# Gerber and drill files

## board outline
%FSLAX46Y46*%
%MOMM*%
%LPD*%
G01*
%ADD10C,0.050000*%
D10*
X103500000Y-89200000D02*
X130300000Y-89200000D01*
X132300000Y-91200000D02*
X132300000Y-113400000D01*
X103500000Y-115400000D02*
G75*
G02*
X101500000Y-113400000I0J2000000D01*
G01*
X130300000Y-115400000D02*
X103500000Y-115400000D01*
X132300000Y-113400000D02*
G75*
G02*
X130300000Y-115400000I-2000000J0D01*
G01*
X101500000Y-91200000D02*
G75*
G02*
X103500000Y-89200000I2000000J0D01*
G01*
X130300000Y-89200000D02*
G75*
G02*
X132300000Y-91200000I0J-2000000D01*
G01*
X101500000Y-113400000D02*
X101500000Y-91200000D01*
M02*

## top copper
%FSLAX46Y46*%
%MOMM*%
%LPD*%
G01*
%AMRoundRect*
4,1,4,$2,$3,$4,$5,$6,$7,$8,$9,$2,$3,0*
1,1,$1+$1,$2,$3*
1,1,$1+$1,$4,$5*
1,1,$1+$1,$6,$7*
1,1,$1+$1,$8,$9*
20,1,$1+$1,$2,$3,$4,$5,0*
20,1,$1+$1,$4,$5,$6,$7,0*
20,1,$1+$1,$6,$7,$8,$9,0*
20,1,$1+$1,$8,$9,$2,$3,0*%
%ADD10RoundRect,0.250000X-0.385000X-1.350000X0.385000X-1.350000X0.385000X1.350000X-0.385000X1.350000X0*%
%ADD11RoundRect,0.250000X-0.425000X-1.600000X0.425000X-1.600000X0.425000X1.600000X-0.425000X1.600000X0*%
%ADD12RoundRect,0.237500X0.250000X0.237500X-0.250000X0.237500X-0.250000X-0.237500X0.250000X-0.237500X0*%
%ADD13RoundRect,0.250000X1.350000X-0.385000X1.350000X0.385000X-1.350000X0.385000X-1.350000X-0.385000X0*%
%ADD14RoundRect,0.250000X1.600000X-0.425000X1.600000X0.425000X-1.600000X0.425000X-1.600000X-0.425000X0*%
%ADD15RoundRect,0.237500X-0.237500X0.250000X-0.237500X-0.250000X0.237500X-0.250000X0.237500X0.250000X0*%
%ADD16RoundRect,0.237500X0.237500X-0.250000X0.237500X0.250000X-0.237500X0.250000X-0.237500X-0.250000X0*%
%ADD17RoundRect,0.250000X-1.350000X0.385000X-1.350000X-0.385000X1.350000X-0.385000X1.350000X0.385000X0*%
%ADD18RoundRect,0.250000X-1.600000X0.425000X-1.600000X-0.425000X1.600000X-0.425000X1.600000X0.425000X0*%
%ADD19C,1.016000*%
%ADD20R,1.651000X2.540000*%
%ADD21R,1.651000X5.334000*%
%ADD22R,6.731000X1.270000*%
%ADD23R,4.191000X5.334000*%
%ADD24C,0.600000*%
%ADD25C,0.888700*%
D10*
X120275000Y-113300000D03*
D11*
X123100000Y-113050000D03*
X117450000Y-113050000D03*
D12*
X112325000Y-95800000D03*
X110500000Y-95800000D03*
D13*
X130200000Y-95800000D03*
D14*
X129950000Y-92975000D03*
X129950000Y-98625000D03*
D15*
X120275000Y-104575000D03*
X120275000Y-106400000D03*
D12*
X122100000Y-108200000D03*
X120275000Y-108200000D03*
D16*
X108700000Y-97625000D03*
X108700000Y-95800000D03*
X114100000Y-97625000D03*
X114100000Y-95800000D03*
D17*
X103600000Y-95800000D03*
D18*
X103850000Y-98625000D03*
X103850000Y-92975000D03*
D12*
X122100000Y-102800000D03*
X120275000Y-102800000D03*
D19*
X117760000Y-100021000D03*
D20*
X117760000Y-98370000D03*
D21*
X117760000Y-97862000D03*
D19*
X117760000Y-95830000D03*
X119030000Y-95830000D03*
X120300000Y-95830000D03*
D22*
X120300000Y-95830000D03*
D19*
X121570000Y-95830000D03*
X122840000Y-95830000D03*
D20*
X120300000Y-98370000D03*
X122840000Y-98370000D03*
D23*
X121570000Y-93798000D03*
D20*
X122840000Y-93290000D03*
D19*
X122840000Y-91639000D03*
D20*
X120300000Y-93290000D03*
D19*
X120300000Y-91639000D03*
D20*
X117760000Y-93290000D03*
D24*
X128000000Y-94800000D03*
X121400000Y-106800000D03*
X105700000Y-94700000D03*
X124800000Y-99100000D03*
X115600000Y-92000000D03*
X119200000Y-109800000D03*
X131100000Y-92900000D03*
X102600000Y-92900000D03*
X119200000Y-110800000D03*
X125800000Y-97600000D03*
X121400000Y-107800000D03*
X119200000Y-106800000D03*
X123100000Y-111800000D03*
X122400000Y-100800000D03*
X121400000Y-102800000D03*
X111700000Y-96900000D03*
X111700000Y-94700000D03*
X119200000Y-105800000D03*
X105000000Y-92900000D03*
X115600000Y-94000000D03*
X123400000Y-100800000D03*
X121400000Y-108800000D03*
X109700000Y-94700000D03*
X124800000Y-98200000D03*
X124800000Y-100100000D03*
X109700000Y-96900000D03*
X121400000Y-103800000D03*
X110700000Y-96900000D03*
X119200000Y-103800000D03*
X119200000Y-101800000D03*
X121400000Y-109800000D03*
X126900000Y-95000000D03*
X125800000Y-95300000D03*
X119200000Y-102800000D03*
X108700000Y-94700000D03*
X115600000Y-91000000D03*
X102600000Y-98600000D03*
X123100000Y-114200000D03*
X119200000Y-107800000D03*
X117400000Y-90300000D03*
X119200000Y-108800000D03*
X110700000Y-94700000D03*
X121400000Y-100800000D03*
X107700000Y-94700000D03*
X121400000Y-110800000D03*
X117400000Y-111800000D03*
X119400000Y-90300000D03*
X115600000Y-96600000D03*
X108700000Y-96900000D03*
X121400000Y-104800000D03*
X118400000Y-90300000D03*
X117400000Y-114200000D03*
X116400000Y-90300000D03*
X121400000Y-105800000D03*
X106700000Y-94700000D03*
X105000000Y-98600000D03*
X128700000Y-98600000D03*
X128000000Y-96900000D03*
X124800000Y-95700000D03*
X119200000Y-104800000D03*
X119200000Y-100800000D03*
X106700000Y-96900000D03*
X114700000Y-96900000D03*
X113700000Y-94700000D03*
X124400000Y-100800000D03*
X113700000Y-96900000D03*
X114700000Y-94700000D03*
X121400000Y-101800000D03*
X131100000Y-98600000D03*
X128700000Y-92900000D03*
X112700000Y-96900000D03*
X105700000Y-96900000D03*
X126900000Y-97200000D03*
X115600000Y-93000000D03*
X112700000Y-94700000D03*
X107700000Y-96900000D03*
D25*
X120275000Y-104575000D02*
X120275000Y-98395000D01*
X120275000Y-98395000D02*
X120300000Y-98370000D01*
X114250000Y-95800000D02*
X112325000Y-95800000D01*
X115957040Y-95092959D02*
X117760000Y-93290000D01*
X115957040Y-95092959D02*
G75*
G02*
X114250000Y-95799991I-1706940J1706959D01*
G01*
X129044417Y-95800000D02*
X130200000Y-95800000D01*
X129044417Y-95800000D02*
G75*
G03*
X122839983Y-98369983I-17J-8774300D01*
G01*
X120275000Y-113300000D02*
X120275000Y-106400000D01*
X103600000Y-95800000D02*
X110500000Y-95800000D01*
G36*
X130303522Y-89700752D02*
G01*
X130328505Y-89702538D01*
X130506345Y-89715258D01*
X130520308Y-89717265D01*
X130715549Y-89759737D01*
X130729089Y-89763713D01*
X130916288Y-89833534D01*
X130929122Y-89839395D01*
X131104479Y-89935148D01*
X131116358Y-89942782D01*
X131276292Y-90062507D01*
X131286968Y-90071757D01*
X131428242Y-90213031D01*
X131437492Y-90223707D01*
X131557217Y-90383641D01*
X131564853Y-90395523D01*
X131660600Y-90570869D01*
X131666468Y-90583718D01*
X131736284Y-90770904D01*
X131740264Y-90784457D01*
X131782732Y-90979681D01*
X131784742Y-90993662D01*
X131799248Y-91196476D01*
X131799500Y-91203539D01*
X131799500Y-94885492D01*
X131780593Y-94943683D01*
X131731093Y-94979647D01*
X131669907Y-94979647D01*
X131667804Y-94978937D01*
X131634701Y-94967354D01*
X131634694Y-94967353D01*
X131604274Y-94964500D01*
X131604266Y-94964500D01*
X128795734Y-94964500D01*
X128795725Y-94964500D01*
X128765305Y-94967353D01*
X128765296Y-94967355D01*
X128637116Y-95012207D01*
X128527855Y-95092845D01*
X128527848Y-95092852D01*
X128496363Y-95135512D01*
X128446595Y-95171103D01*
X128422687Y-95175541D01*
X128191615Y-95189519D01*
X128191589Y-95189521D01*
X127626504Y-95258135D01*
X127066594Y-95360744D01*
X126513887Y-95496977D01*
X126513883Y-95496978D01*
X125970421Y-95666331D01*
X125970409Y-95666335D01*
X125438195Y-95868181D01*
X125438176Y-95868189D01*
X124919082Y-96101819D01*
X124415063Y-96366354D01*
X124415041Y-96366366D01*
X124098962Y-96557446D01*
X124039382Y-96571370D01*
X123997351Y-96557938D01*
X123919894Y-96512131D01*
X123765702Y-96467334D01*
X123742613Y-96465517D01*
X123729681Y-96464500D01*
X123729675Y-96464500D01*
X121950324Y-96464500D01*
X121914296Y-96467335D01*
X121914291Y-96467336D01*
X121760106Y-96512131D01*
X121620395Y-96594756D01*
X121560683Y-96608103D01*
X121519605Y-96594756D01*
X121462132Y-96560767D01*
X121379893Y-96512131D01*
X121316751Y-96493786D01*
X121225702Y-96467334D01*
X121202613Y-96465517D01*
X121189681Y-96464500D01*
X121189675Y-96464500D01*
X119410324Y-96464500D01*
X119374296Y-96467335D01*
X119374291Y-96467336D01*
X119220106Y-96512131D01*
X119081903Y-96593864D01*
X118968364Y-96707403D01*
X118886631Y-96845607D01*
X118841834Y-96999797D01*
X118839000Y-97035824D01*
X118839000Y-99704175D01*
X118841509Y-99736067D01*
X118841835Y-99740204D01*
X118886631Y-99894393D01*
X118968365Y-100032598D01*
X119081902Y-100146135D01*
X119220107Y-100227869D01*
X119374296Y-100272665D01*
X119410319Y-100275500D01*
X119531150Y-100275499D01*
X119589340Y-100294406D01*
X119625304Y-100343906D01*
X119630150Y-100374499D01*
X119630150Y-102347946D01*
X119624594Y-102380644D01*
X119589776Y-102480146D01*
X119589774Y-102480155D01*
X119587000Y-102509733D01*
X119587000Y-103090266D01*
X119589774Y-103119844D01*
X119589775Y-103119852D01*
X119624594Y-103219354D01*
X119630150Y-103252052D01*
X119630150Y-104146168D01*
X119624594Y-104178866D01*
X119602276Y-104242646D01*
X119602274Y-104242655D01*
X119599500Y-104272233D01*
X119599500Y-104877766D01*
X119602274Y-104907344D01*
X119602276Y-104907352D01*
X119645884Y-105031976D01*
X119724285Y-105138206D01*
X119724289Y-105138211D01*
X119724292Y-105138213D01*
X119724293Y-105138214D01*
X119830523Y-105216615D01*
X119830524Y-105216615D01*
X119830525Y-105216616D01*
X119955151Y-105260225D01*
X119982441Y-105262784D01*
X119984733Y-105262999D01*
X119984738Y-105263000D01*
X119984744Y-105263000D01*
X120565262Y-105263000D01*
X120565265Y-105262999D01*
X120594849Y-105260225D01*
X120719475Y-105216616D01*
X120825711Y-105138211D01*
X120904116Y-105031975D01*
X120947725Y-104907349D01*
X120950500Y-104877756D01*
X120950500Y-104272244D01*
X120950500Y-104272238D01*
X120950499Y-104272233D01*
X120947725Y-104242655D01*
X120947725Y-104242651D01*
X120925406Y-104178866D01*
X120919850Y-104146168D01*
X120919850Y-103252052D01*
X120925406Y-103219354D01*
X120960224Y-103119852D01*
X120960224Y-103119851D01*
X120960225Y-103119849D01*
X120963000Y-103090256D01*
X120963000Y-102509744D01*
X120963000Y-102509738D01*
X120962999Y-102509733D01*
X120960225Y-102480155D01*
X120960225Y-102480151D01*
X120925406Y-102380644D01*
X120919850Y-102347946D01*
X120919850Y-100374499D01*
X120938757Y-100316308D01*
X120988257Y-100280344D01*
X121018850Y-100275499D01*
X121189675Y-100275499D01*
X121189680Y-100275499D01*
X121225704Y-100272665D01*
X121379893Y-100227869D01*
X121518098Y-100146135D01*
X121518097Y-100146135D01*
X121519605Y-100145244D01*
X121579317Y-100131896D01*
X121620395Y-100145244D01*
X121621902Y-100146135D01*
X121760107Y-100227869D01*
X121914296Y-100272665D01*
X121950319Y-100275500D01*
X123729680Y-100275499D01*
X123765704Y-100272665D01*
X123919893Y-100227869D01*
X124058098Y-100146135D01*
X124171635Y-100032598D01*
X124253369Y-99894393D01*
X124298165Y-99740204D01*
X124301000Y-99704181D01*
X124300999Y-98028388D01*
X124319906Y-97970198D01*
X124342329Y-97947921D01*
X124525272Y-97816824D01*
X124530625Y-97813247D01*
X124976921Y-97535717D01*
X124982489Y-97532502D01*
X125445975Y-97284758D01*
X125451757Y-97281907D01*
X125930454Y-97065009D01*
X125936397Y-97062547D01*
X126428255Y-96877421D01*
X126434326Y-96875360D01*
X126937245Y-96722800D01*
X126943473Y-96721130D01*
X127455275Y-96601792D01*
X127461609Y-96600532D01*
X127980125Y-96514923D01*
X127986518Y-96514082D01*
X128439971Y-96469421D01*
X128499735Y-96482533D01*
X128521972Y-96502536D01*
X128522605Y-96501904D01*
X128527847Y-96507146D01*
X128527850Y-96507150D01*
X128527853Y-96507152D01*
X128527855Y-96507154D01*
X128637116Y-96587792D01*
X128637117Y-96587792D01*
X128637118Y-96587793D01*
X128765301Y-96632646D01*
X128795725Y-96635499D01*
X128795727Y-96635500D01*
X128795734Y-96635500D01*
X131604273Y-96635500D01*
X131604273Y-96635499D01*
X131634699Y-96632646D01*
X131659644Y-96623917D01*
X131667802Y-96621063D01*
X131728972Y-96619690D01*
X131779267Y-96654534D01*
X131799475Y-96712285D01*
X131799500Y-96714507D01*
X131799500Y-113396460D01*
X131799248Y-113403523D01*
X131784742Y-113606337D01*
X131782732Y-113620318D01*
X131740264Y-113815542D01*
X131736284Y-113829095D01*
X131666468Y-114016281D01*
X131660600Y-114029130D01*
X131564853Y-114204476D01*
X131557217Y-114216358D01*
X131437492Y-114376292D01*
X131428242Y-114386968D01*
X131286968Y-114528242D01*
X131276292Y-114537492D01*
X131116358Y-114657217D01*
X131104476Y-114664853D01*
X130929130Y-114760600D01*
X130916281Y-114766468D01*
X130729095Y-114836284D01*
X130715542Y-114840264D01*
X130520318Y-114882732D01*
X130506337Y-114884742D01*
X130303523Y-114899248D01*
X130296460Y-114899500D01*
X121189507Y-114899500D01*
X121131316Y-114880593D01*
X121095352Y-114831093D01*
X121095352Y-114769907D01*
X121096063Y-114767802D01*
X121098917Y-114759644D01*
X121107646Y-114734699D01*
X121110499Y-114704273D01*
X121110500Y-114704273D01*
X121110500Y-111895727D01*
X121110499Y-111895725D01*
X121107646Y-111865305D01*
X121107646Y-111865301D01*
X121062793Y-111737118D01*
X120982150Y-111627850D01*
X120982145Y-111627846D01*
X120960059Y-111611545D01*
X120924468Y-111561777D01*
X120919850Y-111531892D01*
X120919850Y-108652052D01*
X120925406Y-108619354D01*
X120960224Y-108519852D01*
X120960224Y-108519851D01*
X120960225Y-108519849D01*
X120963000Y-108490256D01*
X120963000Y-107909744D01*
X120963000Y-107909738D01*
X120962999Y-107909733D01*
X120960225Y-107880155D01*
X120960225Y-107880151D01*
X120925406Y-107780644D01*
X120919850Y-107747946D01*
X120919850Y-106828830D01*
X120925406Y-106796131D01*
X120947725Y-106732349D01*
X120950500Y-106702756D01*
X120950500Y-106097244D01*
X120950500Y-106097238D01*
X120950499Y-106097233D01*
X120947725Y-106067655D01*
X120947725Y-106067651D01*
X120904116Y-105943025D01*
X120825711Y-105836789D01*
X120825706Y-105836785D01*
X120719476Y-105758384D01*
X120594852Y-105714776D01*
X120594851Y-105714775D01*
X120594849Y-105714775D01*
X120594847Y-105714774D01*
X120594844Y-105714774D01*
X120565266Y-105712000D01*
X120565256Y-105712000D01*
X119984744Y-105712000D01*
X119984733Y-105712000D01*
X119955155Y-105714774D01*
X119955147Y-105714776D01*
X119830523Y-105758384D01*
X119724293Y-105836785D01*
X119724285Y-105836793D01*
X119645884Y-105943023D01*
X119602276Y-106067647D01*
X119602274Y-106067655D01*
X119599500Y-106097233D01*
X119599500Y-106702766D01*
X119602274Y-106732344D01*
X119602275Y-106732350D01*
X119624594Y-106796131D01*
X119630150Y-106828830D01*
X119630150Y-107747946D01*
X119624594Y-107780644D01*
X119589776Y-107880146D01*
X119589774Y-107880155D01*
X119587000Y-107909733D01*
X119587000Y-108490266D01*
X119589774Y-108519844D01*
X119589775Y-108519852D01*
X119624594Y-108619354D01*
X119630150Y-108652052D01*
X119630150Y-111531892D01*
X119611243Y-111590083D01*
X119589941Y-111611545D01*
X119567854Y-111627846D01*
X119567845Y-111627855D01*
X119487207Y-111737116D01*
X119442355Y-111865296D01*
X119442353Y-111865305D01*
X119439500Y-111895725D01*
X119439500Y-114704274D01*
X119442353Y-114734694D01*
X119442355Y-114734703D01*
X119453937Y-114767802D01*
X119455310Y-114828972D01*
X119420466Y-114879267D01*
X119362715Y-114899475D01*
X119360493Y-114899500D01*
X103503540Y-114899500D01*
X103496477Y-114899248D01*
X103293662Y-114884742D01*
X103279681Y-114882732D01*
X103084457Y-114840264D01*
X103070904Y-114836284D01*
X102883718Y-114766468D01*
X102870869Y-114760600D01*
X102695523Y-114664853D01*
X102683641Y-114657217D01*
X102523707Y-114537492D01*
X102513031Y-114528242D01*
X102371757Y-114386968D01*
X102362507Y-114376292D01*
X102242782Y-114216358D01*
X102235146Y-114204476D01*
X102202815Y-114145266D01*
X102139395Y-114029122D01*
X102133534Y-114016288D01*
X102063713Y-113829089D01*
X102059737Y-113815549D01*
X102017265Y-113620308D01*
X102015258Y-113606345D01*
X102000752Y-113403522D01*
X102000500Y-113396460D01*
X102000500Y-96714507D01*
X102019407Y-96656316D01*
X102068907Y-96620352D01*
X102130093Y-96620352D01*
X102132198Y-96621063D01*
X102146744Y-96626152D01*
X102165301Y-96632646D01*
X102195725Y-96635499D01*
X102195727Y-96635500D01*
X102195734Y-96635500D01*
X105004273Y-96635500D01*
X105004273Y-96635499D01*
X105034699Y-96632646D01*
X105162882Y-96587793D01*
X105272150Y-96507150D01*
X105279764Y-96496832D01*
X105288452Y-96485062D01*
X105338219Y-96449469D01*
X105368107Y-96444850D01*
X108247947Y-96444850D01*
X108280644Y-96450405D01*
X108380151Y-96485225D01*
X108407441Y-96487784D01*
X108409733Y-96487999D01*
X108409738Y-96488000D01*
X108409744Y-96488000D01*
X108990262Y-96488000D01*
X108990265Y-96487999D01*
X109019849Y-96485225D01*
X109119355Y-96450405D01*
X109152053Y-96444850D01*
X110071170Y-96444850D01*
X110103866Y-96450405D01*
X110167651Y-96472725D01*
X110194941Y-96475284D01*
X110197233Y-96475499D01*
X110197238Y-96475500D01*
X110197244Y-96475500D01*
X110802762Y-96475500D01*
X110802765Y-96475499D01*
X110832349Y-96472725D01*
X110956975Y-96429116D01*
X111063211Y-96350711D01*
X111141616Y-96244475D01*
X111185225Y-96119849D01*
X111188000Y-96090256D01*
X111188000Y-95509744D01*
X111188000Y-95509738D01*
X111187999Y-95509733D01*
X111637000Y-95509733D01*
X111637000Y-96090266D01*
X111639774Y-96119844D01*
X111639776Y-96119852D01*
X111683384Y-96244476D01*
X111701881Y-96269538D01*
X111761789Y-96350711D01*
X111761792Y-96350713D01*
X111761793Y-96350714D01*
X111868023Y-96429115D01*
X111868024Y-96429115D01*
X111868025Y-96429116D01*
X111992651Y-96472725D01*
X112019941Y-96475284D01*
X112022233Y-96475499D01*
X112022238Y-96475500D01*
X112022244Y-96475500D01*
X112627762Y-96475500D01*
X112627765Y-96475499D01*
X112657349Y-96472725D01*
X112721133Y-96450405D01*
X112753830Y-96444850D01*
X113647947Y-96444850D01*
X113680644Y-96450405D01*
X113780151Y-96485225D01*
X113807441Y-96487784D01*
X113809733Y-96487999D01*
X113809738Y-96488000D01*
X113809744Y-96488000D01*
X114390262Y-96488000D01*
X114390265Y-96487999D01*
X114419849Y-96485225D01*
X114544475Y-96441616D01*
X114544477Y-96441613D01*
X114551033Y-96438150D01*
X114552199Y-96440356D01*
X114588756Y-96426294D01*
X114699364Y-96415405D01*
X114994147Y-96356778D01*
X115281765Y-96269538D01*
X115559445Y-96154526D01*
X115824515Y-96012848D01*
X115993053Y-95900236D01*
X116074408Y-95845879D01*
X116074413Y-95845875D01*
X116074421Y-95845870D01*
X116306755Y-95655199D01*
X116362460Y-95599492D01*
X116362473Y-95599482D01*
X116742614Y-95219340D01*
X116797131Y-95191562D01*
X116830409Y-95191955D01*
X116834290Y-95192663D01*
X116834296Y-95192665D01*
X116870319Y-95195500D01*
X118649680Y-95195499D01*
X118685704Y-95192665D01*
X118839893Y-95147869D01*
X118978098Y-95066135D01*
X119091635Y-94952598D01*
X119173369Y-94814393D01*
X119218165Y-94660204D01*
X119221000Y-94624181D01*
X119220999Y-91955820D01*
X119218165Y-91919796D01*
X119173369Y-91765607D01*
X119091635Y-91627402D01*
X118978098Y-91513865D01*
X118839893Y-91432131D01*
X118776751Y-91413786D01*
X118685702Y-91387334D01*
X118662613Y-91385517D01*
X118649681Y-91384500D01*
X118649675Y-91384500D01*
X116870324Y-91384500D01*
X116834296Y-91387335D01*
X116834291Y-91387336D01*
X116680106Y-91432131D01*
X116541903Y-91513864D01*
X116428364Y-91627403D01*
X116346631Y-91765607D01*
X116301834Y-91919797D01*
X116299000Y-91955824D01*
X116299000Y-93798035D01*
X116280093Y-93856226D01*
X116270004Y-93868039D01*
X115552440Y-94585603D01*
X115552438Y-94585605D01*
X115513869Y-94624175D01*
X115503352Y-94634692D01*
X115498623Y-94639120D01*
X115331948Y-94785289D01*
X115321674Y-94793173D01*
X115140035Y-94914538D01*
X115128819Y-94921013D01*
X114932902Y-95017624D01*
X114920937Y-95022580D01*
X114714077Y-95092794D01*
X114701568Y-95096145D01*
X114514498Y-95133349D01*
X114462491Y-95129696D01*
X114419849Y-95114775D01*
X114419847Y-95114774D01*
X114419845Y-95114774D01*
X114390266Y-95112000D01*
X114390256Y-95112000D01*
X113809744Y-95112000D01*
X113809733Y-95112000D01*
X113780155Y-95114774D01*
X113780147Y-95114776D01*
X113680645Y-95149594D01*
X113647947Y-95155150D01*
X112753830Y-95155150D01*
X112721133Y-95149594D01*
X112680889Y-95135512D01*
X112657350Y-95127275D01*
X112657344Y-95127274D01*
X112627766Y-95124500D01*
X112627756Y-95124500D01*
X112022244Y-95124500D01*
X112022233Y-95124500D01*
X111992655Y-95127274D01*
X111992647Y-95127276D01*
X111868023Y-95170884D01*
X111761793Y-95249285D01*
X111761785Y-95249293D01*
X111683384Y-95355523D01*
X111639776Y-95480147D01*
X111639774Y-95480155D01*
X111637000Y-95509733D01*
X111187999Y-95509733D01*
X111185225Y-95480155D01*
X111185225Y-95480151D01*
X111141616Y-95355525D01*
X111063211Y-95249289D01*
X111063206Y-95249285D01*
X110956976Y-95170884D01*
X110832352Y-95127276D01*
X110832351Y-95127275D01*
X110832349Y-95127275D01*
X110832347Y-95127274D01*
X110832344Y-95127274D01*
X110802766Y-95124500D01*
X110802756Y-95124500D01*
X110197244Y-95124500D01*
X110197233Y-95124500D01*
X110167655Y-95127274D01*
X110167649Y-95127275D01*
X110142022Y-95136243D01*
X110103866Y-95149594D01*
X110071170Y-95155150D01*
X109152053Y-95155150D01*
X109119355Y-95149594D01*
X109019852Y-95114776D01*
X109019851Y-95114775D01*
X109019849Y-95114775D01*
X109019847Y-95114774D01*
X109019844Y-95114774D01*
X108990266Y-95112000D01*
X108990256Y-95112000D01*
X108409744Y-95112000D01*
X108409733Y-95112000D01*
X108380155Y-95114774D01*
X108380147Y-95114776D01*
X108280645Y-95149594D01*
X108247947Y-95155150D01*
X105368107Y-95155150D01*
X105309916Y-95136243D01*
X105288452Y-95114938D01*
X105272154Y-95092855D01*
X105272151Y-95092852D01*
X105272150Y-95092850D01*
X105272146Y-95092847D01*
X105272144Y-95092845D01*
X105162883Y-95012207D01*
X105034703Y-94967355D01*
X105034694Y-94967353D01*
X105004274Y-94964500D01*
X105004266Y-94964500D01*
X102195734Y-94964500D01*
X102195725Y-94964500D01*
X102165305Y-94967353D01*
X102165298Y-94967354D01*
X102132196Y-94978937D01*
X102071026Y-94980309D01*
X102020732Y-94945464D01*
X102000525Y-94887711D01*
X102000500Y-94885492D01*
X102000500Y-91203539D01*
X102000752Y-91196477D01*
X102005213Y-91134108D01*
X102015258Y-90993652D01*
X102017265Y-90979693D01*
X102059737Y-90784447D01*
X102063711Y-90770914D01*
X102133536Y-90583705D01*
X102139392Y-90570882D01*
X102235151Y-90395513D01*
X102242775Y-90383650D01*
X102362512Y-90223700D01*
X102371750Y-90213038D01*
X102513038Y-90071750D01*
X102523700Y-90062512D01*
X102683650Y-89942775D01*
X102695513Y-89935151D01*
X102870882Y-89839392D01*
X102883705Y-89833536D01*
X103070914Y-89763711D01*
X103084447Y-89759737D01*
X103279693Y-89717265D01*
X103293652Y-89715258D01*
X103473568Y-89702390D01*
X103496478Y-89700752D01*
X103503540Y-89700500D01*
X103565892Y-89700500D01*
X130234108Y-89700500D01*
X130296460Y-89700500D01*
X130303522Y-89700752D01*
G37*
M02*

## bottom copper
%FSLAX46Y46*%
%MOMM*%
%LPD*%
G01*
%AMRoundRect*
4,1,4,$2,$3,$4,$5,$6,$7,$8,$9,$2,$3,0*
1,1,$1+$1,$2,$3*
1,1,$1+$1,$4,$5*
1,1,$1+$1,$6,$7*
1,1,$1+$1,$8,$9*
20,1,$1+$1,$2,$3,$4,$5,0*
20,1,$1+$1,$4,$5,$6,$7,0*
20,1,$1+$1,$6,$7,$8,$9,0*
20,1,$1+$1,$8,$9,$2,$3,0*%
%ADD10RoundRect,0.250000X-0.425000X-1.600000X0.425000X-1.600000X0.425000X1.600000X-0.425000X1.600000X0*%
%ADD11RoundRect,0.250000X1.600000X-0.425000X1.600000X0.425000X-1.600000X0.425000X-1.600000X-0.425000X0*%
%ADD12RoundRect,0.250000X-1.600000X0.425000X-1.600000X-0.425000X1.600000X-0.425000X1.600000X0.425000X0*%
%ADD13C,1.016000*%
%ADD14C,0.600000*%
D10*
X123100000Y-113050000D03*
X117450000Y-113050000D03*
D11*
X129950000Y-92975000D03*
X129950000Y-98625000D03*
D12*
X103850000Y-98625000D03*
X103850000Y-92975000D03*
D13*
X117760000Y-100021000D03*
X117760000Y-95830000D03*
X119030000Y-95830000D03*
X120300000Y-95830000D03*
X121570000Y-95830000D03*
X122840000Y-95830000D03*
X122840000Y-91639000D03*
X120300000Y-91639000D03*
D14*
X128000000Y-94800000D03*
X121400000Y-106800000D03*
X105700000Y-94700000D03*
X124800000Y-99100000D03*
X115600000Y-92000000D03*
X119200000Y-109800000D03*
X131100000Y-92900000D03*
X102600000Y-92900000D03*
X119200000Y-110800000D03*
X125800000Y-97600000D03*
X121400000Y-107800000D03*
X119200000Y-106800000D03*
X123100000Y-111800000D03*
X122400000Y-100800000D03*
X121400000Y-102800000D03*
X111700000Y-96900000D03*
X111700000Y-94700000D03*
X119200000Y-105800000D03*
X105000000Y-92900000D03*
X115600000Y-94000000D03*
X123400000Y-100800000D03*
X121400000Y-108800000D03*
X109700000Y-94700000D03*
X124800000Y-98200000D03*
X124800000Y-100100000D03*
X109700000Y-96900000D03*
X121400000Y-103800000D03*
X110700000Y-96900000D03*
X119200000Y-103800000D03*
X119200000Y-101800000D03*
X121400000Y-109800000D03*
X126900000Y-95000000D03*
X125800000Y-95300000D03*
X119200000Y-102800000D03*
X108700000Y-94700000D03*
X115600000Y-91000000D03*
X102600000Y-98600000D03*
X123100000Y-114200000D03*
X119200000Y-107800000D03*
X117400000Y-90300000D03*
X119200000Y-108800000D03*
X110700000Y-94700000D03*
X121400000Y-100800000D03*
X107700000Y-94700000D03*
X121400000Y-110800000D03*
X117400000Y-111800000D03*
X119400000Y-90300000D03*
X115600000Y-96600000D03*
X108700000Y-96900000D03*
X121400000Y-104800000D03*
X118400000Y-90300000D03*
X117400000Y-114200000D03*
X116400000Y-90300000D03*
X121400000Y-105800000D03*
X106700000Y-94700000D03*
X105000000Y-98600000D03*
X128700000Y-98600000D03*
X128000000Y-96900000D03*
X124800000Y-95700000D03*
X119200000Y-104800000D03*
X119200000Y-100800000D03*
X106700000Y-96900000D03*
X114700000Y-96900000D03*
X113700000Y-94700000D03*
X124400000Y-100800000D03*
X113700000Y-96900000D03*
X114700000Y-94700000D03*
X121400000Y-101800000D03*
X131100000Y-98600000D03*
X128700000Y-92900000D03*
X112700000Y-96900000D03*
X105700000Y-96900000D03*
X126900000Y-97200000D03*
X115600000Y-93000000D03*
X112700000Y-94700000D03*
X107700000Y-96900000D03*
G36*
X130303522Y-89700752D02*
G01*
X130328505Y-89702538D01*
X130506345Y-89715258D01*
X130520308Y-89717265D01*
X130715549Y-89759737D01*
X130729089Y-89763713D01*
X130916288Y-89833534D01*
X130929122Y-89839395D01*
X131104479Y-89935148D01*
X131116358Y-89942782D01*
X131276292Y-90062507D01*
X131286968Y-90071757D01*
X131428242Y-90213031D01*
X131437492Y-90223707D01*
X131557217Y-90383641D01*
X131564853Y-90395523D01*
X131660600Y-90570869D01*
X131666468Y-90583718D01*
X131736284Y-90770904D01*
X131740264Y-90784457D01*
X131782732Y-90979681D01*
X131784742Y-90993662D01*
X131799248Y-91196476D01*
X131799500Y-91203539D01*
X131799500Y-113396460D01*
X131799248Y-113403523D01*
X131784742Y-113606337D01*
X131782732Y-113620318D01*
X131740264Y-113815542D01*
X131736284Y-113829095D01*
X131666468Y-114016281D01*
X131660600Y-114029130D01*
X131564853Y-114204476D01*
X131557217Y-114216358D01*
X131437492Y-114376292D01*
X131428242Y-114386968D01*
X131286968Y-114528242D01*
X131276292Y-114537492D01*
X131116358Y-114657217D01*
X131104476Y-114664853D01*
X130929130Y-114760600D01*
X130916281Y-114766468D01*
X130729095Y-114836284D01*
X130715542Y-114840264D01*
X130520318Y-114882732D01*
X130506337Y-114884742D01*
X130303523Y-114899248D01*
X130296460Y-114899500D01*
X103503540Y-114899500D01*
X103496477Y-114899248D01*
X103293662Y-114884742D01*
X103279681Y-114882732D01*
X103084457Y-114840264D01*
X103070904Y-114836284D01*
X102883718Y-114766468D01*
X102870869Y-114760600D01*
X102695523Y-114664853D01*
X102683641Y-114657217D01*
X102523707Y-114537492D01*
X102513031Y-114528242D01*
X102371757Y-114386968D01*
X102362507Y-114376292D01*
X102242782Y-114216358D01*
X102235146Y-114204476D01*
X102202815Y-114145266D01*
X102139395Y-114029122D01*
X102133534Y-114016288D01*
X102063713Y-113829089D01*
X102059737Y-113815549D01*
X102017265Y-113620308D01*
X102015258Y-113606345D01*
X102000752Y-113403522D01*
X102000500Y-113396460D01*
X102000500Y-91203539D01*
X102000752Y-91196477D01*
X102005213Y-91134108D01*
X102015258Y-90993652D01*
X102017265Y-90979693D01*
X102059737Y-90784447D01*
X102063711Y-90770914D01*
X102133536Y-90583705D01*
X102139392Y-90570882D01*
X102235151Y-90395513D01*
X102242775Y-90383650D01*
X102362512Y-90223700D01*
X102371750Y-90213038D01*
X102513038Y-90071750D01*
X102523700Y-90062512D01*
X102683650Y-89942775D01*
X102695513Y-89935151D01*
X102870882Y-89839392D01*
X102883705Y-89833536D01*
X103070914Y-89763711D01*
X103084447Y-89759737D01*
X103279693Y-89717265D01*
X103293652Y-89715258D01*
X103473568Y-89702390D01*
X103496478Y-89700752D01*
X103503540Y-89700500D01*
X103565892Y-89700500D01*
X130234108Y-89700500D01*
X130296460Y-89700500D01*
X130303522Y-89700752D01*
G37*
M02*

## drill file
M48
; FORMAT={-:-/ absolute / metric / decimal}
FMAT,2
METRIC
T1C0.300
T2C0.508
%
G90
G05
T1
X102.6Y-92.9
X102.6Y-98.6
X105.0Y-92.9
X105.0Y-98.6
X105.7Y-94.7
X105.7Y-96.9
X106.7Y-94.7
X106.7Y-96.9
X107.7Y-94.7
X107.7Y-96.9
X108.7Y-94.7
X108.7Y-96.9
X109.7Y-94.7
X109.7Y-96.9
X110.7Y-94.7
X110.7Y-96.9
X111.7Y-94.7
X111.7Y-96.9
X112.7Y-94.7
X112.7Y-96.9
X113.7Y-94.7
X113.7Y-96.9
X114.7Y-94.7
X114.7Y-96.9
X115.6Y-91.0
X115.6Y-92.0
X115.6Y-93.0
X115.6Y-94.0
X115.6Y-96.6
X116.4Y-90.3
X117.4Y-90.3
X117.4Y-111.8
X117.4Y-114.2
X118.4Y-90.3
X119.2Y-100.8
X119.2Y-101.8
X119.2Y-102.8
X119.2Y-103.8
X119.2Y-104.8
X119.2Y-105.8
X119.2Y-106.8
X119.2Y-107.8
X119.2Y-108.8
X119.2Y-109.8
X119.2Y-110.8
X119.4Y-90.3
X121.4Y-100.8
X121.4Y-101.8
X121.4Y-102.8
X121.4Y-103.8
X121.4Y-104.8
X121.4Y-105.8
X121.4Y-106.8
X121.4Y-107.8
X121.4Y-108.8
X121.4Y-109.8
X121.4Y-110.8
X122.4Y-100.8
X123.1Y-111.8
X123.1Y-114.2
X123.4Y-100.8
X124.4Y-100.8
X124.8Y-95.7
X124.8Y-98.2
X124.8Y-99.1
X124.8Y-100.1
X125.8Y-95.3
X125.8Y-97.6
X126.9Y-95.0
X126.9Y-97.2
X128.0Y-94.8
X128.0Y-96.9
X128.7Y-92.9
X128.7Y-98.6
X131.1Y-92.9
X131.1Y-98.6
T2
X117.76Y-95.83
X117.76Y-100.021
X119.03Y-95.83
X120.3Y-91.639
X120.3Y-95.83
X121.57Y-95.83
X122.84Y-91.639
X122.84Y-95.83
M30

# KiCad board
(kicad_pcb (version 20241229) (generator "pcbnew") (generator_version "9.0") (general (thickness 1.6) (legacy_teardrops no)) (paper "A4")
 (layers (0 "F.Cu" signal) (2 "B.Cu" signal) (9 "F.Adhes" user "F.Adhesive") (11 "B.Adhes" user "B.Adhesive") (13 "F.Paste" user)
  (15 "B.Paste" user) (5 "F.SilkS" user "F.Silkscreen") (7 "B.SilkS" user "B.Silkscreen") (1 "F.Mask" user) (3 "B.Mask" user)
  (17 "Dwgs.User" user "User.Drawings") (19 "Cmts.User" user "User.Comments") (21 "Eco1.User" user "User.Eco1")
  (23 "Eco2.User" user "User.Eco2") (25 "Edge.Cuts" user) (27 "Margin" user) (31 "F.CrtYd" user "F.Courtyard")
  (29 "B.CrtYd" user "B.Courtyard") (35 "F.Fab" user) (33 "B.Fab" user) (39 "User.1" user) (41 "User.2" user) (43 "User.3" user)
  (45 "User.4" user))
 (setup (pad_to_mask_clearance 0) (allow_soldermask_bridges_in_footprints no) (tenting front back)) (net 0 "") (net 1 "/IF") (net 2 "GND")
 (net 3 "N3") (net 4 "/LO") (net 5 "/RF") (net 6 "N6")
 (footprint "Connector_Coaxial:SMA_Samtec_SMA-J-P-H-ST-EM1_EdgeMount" (layer "F.Cu") (at 120.275 113.3 -90)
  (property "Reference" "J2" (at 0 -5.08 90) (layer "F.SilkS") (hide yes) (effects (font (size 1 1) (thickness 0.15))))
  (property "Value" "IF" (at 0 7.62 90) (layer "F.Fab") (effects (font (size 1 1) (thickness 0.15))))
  (pad "1" smd roundrect (at 0 0) (size 1.27 3.2) (layers "F.Cu" "F.Mask") (roundrect_rratio 0.1968503937) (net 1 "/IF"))
  (pad "2" smd roundrect (at -0.25 -2.825) (size 1.35 3.7) (layers "F.Cu" "F.Mask") (roundrect_rratio 0.1851851852) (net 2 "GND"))
  (pad "2" smd roundrect (at -0.25 -2.825) (size 1.35 3.7) (layers "B.Cu" "B.Mask") (roundrect_rratio 0.1851851852) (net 2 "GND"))
  (pad "2" smd roundrect (at -0.25 2.825) (size 1.35 3.7) (layers "F.Cu" "F.Mask") (roundrect_rratio 0.1851851852) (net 2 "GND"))
  (pad "2" smd roundrect (at -0.25 2.825) (size 1.35 3.7) (layers "B.Cu" "B.Mask") (roundrect_rratio 0.1851851852) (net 2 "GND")))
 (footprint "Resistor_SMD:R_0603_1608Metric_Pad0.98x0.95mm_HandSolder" (layer "F.Cu") (at 111.4125 95.8 180)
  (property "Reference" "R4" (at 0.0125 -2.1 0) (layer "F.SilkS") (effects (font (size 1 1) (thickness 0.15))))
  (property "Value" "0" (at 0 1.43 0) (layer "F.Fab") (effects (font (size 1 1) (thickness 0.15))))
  (pad "1" smd roundrect (at -0.9125 0 180) (size 0.975 0.95) (layers "F.Cu" "F.Mask" "F.Paste") (roundrect_rratio 0.25) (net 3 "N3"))
  (pad "2" smd roundrect (at 0.9125 0 180) (size 0.975 0.95) (layers "F.Cu" "F.Mask" "F.Paste") (roundrect_rratio 0.25) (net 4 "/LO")))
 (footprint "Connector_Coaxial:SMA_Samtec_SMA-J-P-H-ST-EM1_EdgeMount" (layer "F.Cu") (at 130.2 95.8)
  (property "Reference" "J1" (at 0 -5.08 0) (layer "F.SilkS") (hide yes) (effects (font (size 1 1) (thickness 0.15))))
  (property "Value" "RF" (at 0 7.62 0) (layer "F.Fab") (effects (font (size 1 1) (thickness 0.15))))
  (pad "1" smd roundrect (at 0 0 90) (size 1.27 3.2) (layers "F.Cu" "F.Mask") (roundrect_rratio 0.1968503937) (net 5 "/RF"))
  (pad "2" smd roundrect (at -0.25 -2.825 90) (size 1.35 3.7) (layers "F.Cu" "F.Mask") (roundrect_rratio 0.1851851852) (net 2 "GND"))
  (pad "2" smd roundrect (at -0.25 -2.825 90) (size 1.35 3.7) (layers "B.Cu" "B.Mask") (roundrect_rratio 0.1851851852) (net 2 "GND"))
  (pad "2" smd roundrect (at -0.25 2.825 90) (size 1.35 3.7) (layers "F.Cu" "F.Mask") (roundrect_rratio 0.1851851852) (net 2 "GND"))
  (pad "2" smd roundrect (at -0.25 2.825 90) (size 1.35 3.7) (layers "B.Cu" "B.Mask") (roundrect_rratio 0.1851851852) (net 2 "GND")))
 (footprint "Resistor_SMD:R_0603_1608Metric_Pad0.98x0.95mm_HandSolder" (layer "F.Cu") (at 120.275 105.4875 -90)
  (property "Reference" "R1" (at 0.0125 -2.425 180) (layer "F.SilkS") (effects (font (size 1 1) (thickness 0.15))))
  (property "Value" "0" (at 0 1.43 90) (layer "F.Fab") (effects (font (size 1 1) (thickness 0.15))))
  (pad "1" smd roundrect (at -0.9125 0 270) (size 0.975 0.95) (layers "F.Cu" "F.Mask" "F.Paste") (roundrect_rratio 0.25) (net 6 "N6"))
  (pad "2" smd roundrect (at 0.9125 0 270) (size 0.975 0.95) (layers "F.Cu" "F.Mask" "F.Paste") (roundrect_rratio 0.25) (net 1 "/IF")))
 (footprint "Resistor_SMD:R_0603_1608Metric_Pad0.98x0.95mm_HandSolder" (layer "F.Cu") (at 121.1875 108.2 180)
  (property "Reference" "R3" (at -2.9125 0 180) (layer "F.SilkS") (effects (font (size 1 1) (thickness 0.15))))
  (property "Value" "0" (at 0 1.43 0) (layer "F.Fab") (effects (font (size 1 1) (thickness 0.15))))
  (pad "1" smd roundrect (at -0.9125 0 180) (size 0.975 0.95) (layers "F.Cu" "F.Mask" "F.Paste") (roundrect_rratio 0.25) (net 2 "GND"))
  (pad "2" smd roundrect (at 0.9125 0 180) (size 0.975 0.95) (layers "F.Cu" "F.Mask" "F.Paste") (roundrect_rratio 0.25) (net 1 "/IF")))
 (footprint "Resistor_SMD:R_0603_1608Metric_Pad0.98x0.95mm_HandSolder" (layer "F.Cu") (at 108.7 96.7125 90)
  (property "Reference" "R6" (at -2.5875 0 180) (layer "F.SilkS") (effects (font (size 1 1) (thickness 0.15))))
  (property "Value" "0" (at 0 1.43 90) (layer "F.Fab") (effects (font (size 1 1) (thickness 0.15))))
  (pad "1" smd roundrect (at -0.9125 0 90) (size 0.975 0.95) (layers "F.Cu" "F.Mask" "F.Paste") (roundrect_rratio 0.25) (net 2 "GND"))
  (pad "2" smd roundrect (at 0.9125 0 90) (size 0.975 0.95) (layers "F.Cu" "F.Mask" "F.Paste") (roundrect_rratio 0.25) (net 4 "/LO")))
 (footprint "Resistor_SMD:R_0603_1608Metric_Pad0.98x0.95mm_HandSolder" (layer "F.Cu") (at 114.1 96.7125 90)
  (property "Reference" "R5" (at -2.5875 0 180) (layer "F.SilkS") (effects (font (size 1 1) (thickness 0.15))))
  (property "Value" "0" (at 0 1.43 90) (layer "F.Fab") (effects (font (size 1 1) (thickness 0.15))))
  (pad "1" smd roundrect (at -0.9125 0 90) (size 0.975 0.95) (layers "F.Cu" "F.Mask" "F.Paste") (roundrect_rratio 0.25) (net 2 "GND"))
  (pad "2" smd roundrect (at 0.9125 0 90) (size 0.975 0.95) (layers "F.Cu" "F.Mask" "F.Paste") (roundrect_rratio 0.25) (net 3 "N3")))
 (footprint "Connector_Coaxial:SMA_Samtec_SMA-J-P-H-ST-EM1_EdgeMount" (layer "F.Cu") (at 103.6 95.8 180)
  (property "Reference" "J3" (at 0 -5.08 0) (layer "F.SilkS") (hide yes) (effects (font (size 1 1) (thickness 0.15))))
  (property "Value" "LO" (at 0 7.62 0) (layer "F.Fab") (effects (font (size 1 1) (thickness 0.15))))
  (pad "1" smd roundrect (at 0 0 270) (size 1.27 3.2) (layers "F.Cu" "F.Mask") (roundrect_rratio 0.1968503937) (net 4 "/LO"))
  (pad "2" smd roundrect (at -0.25 -2.825 270) (size 1.35 3.7) (layers "F.Cu" "F.Mask") (roundrect_rratio 0.1851851852) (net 2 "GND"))
  (pad "2" smd roundrect (at -0.25 -2.825 270) (size 1.35 3.7) (layers "B.Cu" "B.Mask") (roundrect_rratio 0.1851851852) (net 2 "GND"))
  (pad "2" smd roundrect (at -0.25 2.825 270) (size 1.35 3.7) (layers "F.Cu" "F.Mask") (roundrect_rratio 0.1851851852) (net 2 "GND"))
  (pad "2" smd roundrect (at -0.25 2.825 270) (size 1.35 3.7) (layers "B.Cu" "B.Mask") (roundrect_rratio 0.1851851852) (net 2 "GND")))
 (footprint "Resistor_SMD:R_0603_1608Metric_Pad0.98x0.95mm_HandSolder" (layer "F.Cu") (at 121.1875 102.8 180)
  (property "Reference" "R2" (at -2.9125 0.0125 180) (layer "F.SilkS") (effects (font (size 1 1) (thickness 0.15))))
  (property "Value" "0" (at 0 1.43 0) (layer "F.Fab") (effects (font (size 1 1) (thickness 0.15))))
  (pad "1" smd roundrect (at -0.9125 0 180) (size 0.975 0.95) (layers "F.Cu" "F.Mask" "F.Paste") (roundrect_rratio 0.25) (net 2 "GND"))
  (pad "2" smd roundrect (at 0.9125 0 180) (size 0.975 0.95) (layers "F.Cu" "F.Mask" "F.Paste") (roundrect_rratio 0.25) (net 6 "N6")))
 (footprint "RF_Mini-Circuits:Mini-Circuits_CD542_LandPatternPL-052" (layer "F.Cu") (at 120.3 95.83 90)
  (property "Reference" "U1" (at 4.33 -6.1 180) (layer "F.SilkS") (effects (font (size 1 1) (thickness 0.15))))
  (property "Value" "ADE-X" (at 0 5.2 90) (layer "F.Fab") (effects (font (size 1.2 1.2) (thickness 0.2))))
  (pad "1" thru_hole circle (at -4.191 -2.54 90) (size 1.016 1.016) (drill 0.508) (layers "*.Cu") (remove_unused_layers no) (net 2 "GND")
   (zone_connect 2))
  (pad "1" smd rect (at -2.54 -2.54 90) (size 2.54 1.651) (layers "F.Cu" "F.Mask" "F.Paste") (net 2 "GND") (zone_connect 2))
  (pad "1" smd rect (at -2.032 -2.54 90) (size 5.334 1.651) (layers "F.Cu") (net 2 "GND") (zone_connect 2))
  (pad "1" thru_hole circle (at 0 -2.54 90) (size 1.016 1.016) (drill 0.508) (layers "*.Cu") (remove_unused_layers no) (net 2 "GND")
   (zone_connect 2))
  (pad "1" thru_hole circle (at 0 -1.27 90) (size 1.016 1.016) (drill 0.508) (layers "*.Cu") (remove_unused_layers no) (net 2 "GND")
   (zone_connect 2))
  (pad "1" thru_hole circle (at 0 0 90) (size 1.016 1.016) (drill 0.508) (layers "*.Cu") (remove_unused_layers no) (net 2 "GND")
   (zone_connect 2))
  (pad "1" smd rect (at 0 0 90) (size 1.27 6.731) (layers "F.Cu") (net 2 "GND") (zone_connect 2))
  (pad "1" thru_hole circle (at 0 1.27 90) (size 1.016 1.016) (drill 0.508) (layers "*.Cu") (remove_unused_layers no) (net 2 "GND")
   (zone_connect 2))
  (pad "1" thru_hole circle (at 0 2.54 90) (size 1.016 1.016) (drill 0.508) (layers "*.Cu") (remove_unused_layers no) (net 2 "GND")
   (zone_connect 2))
  (pad "2" smd rect (at -2.54 0 90) (size 2.54 1.651) (layers "F.Cu" "F.Mask" "F.Paste") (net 6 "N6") (clearance 0.635))
  (pad "3" smd rect (at -2.54 2.54 90) (size 2.54 1.651) (layers "F.Cu" "F.Mask" "F.Paste") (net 5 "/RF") (clearance 0.635))
  (pad "4" smd rect (at 2.032 1.27 90) (size 5.334 4.191) (layers "F.Cu") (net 2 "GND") (zone_connect 2))
  (pad "4" smd rect (at 2.54 2.54 90) (size 2.54 1.651) (layers "F.Cu" "F.Mask" "F.Paste") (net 2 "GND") (zone_connect 2))
  (pad "4" thru_hole circle (at 4.191 2.54 90) (size 1.016 1.016) (drill 0.508) (layers "*.Cu") (remove_unused_layers no) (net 2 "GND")
   (zone_connect 2))
  (pad "5" smd rect (at 2.54 0 90) (size 2.54 1.651) (layers "F.Cu" "F.Mask" "F.Paste") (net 2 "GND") (zone_connect 2))
  (pad "5" thru_hole circle (at 4.191 0 90) (size 1.016 1.016) (drill 0.508) (layers "*.Cu") (remove_unused_layers no) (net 2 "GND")
   (zone_connect 2))
  (pad "6" smd rect (at 2.54 -2.54 90) (size 2.54 1.651) (layers "F.Cu" "F.Mask" "F.Paste") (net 3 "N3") (clearance 0.635)))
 (gr_line (start 103.5 89.2) (end 130.3 89.2) (stroke (width 0.05) (type default)) (layer "Edge.Cuts"))
 (gr_line (start 132.3 91.2) (end 132.3 113.4) (stroke (width 0.05) (type default)) (layer "Edge.Cuts"))
 (gr_arc (start 103.5 115.4) (mid 102.085786 114.814214) (end 101.5 113.4) (stroke (width 0.05) (type default)) (layer "Edge.Cuts"))
 (gr_line (start 130.3 115.4) (end 103.5 115.4) (stroke (width 0.05) (type default)) (layer "Edge.Cuts"))
 (gr_arc (start 132.3 113.4) (mid 131.714214 114.814214) (end 130.3 115.4) (stroke (width 0.05) (type default)) (layer "Edge.Cuts"))
 (gr_arc (start 101.5 91.2) (mid 102.085786 89.785786) (end 103.5 89.2) (stroke (width 0.05) (type default)) (layer "Edge.Cuts"))
 (gr_arc (start 130.3 89.2) (mid 131.714214 89.785786) (end 132.3 91.2) (stroke (width 0.05) (type default)) (layer "Edge.Cuts"))
 (gr_line (start 101.5 113.4) (end 101.5 91.2) (stroke (width 0.05) (type default)) (layer "Edge.Cuts"))
 (via (at 128 94.8) (size 0.6) (drill 0.3) (layers "F.Cu" "B.Cu") (free yes) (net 2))
 (via (at 121.4 106.8) (size 0.6) (drill 0.3) (layers "F.Cu" "B.Cu") (free yes) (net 2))
 (via (at 105.7 94.7) (size 0.6) (drill 0.3) (layers "F.Cu" "B.Cu") (free yes) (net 2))
 (via (at 124.8 99.1) (size 0.6) (drill 0.3) (layers "F.Cu" "B.Cu") (free yes) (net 2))
 (via (at 115.6 92) (size 0.6) (drill 0.3) (layers "F.Cu" "B.Cu") (free yes) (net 2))
 (via (at 119.2 109.8) (size 0.6) (drill 0.3) (layers "F.Cu" "B.Cu") (free yes) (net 2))
 (via (at 131.1 92.9) (size 0.6) (drill 0.3) (layers "F.Cu" "B.Cu") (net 2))
 (via (at 102.6 92.9) (size 0.6) (drill 0.3) (layers "F.Cu" "B.Cu") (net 2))
 (via (at 119.2 110.8) (size 0.6) (drill 0.3) (layers "F.Cu" "B.Cu") (free yes) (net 2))
 (via (at 125.8 97.6) (size 0.6) (drill 0.3) (layers "F.Cu" "B.Cu") (free yes) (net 2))
 (via (at 121.4 107.8) (size 0.6) (drill 0.3) (layers "F.Cu" "B.Cu") (free yes) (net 2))
 (via (at 119.2 106.8) (size 0.6) (drill 0.3) (layers "F.Cu" "B.Cu") (free yes) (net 2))
 (via (at 123.1 111.8) (size 0.6) (drill 0.3) (layers "F.Cu" "B.Cu") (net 2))
 (via (at 122.4 100.8) (size 0.6) (drill 0.3) (layers "F.Cu" "B.Cu") (free yes) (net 2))
 (via (at 121.4 102.8) (size 0.6) (drill 0.3) (layers "F.Cu" "B.Cu") (free yes) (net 2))
 (via (at 111.7 96.9) (size 0.6) (drill 0.3) (layers "F.Cu" "B.Cu") (free yes) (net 2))
 (via (at 111.7 94.7) (size 0.6) (drill 0.3) (layers "F.Cu" "B.Cu") (free yes) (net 2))
 (via (at 119.2 105.8) (size 0.6) (drill 0.3) (layers "F.Cu" "B.Cu") (free yes) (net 2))
 (via (at 105 92.9) (size 0.6) (drill 0.3) (layers "F.Cu" "B.Cu") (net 2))
 (via (at 115.6 94) (size 0.6) (drill 0.3) (layers "F.Cu" "B.Cu") (free yes) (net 2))
 (via (at 123.4 100.8) (size 0.6) (drill 0.3) (layers "F.Cu" "B.Cu") (free yes) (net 2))
 (via (at 121.4 108.8) (size 0.6) (drill 0.3) (layers "F.Cu" "B.Cu") (free yes) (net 2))
 (via (at 109.7 94.7) (size 0.6) (drill 0.3) (layers "F.Cu" "B.Cu") (free yes) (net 2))
 (via (at 124.8 98.2) (size 0.6) (drill 0.3) (layers "F.Cu" "B.Cu") (free yes) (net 2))
 (via (at 124.8 100.1) (size 0.6) (drill 0.3) (layers "F.Cu" "B.Cu") (free yes) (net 2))
 (via (at 109.7 96.9) (size 0.6) (drill 0.3) (layers "F.Cu" "B.Cu") (free yes) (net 2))
 (via (at 121.4 103.8) (size 0.6) (drill 0.3) (layers "F.Cu" "B.Cu") (free yes) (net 2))
 (via (at 110.7 96.9) (size 0.6) (drill 0.3) (layers "F.Cu" "B.Cu") (free yes) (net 2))
 (via (at 119.2 103.8) (size 0.6) (drill 0.3) (layers "F.Cu" "B.Cu") (free yes) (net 2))
 (via (at 119.2 101.8) (size 0.6) (drill 0.3) (layers "F.Cu" "B.Cu") (free yes) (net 2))
 (via (at 121.4 109.8) (size 0.6) (drill 0.3) (layers "F.Cu" "B.Cu") (free yes) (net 2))
 (via (at 126.9 95) (size 0.6) (drill 0.3) (layers "F.Cu" "B.Cu") (free yes) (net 2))
 (via (at 125.8 95.3) (size 0.6) (drill 0.3) (layers "F.Cu" "B.Cu") (free yes) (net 2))
 (via (at 119.2 102.8) (size 0.6) (drill 0.3) (layers "F.Cu" "B.Cu") (free yes) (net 2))
 (via (at 108.7 94.7) (size 0.6) (drill 0.3) (layers "F.Cu" "B.Cu") (free yes) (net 2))
 (via (at 115.6 91) (size 0.6) (drill 0.3) (layers "F.Cu" "B.Cu") (free yes) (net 2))
 (via (at 102.6 98.6) (size 0.6) (drill 0.3) (layers "F.Cu" "B.Cu") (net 2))
 (via (at 123.1 114.2) (size 0.6) (drill 0.3) (layers "F.Cu" "B.Cu") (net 2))
 (via (at 119.2 107.8) (size 0.6) (drill 0.3) (layers "F.Cu" "B.Cu") (free yes) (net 2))
 (via (at 117.4 90.3) (size 0.6) (drill 0.3) (layers "F.Cu" "B.Cu") (free yes) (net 2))
 (via (at 119.2 108.8) (size 0.6) (drill 0.3) (layers "F.Cu" "B.Cu") (free yes) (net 2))
 (via (at 110.7 94.7) (size 0.6) (drill 0.3) (layers "F.Cu" "B.Cu") (free yes) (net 2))
 (via (at 121.4 100.8) (size 0.6) (drill 0.3) (layers "F.Cu" "B.Cu") (free yes) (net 2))
 (via (at 107.7 94.7) (size 0.6) (drill 0.3) (layers "F.Cu" "B.Cu") (free yes) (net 2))
 (via (at 121.4 110.8) (size 0.6) (drill 0.3) (layers "F.Cu" "B.Cu") (free yes) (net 2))
 (via (at 117.4 111.8) (size 0.6) (drill 0.3) (layers "F.Cu" "B.Cu") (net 2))
 (via (at 119.4 90.3) (size 0.6) (drill 0.3) (layers "F.Cu" "B.Cu") (free yes) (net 2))
 (via (at 115.6 96.6) (size 0.6) (drill 0.3) (layers "F.Cu" "B.Cu") (free yes) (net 2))
 (via (at 108.7 96.9) (size 0.6) (drill 0.3) (layers "F.Cu" "B.Cu") (free yes) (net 2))
 (via (at 121.4 104.8) (size 0.6) (drill 0.3) (layers "F.Cu" "B.Cu") (free yes) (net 2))
 (via (at 118.4 90.3) (size 0.6) (drill 0.3) (layers "F.Cu" "B.Cu") (free yes) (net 2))
 (via (at 117.4 114.2) (size 0.6) (drill 0.3) (layers "F.Cu" "B.Cu") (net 2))
 (via (at 116.4 90.3) (size 0.6) (drill 0.3) (layers "F.Cu" "B.Cu") (free yes) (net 2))
 (via (at 121.4 105.8) (size 0.6) (drill 0.3) (layers "F.Cu" "B.Cu") (free yes) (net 2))
 (via (at 106.7 94.7) (size 0.6) (drill 0.3) (layers "F.Cu" "B.Cu") (free yes) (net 2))
 (via (at 105 98.6) (size 0.6) (drill 0.3) (layers "F.Cu" "B.Cu") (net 2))
 (via (at 128.7 98.6) (size 0.6) (drill 0.3) (layers "F.Cu" "B.Cu") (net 2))
 (via (at 128 96.9) (size 0.6) (drill 0.3) (layers "F.Cu" "B.Cu") (free yes) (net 2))
 (via (at 124.8 95.7) (size 0.6) (drill 0.3) (layers "F.Cu" "B.Cu") (free yes) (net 2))
 (via (at 119.2 104.8) (size 0.6) (drill 0.3) (layers "F.Cu" "B.Cu") (free yes) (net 2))
 (via (at 119.2 100.8) (size 0.6) (drill 0.3) (layers "F.Cu" "B.Cu") (free yes) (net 2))
 (via (at 106.7 96.9) (size 0.6) (drill 0.3) (layers "F.Cu" "B.Cu") (free yes) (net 2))
 (via (at 114.7 96.9) (size 0.6) (drill 0.3) (layers "F.Cu" "B.Cu") (free yes) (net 2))
 (via (at 113.7 94.7) (size 0.6) (drill 0.3) (layers "F.Cu" "B.Cu") (free yes) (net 2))
 (via (at 124.4 100.8) (size 0.6) (drill 0.3) (layers "F.Cu" "B.Cu") (free yes) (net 2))
 (via (at 113.7 96.9) (size 0.6) (drill 0.3) (layers "F.Cu" "B.Cu") (free yes) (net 2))
 (via (at 114.7 94.7) (size 0.6) (drill 0.3) (layers "F.Cu" "B.Cu") (free yes) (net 2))
 (via (at 121.4 101.8) (size 0.6) (drill 0.3) (layers "F.Cu" "B.Cu") (free yes) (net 2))
 (via (at 131.1 98.6) (size 0.6) (drill 0.3) (layers "F.Cu" "B.Cu") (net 2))
 (via (at 128.7 92.9) (size 0.6) (drill 0.3) (layers "F.Cu" "B.Cu") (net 2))
 (via (at 112.7 96.9) (size 0.6) (drill 0.3) (layers "F.Cu" "B.Cu") (free yes) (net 2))
 (via (at 105.7 96.9) (size 0.6) (drill 0.3) (layers "F.Cu" "B.Cu") (free yes) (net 2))
 (via (at 126.9 97.2) (size 0.6) (drill 0.3) (layers "F.Cu" "B.Cu") (free yes) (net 2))
 (via (at 115.6 93) (size 0.6) (drill 0.3) (layers "F.Cu" "B.Cu") (free yes) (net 2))
 (via (at 112.7 94.7) (size 0.6) (drill 0.3) (layers "F.Cu" "B.Cu") (free yes) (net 2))
 (via (at 107.7 96.9) (size 0.6) (drill 0.3) (layers "F.Cu" "B.Cu") (free yes) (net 2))
 (segment (start 120.275 104.575) (end 120.275 98.395) (width 0.8887) (layer "F.Cu") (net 6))
 (segment (start 120.275 98.395) (end 120.3 98.37) (width 0.8887) (layer "F.Cu") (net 6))
 (segment (start 114.25 95.8) (end 112.325 95.8) (width 0.8887) (layer "F.Cu") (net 3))
 (segment (start 115.95704 95.092959) (end 117.76 93.29) (width 0.8887) (layer "F.Cu") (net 3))
 (arc (start 115.95704 95.092959) (mid 115.173886 95.616246) (end 114.25 95.799999) (width 0.8887) (layer "F.Cu") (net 3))
 (segment (start 129.044417 95.8) (end 130.2 95.8) (width 0.8887) (layer "F.Cu") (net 5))
 (arc (start 129.044417 95.8) (mid 125.686621 96.467914) (end 122.84 98.37) (width 0.8887) (layer "F.Cu") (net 5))
 (segment (start 120.275 113.3) (end 120.275 106.4) (width 0.8887) (layer "F.Cu") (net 1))
 (segment (start 103.6 95.8) (end 110.5 95.8) (width 0.8887) (layer "F.Cu") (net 4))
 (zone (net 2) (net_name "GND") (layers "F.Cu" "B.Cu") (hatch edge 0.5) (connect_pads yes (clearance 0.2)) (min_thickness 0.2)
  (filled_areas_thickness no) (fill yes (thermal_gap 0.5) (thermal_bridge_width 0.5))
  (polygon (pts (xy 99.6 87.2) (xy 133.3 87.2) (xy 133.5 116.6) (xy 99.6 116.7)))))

